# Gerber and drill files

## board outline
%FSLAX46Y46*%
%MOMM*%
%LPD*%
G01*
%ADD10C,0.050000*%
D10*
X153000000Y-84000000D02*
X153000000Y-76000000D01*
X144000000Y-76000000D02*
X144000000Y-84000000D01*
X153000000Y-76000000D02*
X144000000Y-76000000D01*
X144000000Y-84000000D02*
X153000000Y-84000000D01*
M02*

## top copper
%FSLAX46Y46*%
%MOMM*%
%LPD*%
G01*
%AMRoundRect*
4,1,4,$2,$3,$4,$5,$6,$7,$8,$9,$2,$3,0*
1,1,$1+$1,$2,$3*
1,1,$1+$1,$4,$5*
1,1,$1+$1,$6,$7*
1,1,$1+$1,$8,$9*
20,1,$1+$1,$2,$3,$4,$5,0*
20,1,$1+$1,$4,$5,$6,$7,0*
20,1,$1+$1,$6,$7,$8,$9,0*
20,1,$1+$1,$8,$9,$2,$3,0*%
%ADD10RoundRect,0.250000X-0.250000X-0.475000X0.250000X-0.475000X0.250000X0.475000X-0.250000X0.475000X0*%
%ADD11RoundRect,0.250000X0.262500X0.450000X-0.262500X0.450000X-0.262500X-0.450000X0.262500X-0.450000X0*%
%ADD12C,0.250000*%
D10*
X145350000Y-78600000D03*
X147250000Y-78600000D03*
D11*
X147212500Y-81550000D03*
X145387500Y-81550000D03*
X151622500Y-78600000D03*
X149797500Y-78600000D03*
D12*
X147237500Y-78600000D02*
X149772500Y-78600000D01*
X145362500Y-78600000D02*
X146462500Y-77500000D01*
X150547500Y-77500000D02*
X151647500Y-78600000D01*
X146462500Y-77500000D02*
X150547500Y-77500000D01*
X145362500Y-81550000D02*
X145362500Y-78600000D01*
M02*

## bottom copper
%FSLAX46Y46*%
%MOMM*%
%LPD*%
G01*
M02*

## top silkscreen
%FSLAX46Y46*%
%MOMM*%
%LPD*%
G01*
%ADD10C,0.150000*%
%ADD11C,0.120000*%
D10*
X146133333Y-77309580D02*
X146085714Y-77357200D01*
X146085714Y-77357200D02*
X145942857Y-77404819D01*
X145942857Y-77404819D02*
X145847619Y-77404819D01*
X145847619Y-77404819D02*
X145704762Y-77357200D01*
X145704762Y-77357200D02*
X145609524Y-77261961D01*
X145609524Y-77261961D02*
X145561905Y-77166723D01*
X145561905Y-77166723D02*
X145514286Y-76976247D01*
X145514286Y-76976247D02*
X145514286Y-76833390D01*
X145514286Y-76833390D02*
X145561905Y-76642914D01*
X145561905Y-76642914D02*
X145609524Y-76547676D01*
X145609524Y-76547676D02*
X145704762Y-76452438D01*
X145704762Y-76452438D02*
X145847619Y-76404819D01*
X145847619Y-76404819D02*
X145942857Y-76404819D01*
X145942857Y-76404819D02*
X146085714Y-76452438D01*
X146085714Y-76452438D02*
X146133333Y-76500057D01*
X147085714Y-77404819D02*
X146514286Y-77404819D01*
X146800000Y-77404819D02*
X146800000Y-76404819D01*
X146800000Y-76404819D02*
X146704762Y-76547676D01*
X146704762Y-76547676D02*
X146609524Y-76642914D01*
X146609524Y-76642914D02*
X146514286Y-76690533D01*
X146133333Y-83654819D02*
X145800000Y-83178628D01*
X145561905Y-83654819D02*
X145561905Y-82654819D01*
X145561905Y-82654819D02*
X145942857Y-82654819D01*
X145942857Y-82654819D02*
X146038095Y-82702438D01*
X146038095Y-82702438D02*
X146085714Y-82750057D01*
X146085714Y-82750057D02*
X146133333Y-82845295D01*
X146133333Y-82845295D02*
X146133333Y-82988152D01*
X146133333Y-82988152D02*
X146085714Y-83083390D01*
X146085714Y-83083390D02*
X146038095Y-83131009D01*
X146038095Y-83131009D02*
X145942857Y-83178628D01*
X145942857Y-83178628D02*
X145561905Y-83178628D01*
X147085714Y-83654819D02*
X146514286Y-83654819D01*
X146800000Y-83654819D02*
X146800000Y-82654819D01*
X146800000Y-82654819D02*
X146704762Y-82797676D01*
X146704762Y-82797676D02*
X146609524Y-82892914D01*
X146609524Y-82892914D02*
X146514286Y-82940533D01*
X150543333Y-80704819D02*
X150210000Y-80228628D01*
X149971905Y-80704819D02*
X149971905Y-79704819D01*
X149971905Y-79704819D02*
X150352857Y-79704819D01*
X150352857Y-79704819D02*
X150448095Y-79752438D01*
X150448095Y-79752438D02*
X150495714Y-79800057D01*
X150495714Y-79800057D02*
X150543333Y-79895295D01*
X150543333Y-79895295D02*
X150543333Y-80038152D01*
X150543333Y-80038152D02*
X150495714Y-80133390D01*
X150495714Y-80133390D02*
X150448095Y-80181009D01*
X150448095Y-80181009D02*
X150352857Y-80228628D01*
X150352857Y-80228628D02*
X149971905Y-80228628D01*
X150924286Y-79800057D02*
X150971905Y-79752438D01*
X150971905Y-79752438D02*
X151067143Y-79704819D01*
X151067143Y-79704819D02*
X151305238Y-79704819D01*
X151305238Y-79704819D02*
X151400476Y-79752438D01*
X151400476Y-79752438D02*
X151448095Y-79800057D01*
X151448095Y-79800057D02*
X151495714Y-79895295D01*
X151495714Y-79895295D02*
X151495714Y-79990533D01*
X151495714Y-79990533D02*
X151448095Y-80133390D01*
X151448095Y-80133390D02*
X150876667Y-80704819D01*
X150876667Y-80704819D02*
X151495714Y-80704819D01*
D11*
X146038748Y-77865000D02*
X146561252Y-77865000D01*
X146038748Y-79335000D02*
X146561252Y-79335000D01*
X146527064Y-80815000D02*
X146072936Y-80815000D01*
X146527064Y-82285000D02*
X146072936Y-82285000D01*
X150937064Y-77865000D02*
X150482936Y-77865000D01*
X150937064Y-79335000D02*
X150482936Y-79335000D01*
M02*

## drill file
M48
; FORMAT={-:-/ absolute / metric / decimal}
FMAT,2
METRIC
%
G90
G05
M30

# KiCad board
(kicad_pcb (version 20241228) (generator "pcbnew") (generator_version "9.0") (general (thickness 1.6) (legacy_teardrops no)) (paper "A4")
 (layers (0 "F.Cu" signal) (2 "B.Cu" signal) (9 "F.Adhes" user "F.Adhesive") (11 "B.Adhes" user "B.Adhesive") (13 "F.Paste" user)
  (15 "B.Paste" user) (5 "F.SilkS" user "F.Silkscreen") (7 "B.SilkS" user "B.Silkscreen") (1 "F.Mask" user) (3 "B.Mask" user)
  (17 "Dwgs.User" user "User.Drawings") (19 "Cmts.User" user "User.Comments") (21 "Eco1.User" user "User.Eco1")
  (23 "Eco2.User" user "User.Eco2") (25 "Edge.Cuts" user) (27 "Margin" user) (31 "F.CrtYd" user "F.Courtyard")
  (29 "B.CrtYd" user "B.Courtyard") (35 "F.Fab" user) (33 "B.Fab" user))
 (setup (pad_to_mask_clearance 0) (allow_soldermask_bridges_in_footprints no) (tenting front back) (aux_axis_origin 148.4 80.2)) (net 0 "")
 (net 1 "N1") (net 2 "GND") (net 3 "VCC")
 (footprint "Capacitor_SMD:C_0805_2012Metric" (layer "F.Cu") (at 146.3 78.6)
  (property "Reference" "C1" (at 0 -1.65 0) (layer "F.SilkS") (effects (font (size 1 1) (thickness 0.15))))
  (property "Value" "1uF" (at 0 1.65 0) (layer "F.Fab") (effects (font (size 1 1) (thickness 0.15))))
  (fp_line (start -0.261252 -0.735) (end 0.261252 -0.735) (stroke (width 0.12) (type solid)) (layer "F.SilkS"))
  (fp_line (start -0.261252 0.735) (end 0.261252 0.735) (stroke (width 0.12) (type solid)) (layer "F.SilkS"))
  (pad "1" smd roundrect (at -0.95 0) (size 1 1.45) (layers "F.Cu" "F.Mask" "F.Paste") (roundrect_rratio 0.25) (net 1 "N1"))
  (pad "2" smd roundrect (at 0.95 0) (size 1 1.45) (layers "F.Cu" "F.Mask" "F.Paste") (roundrect_rratio 0.25) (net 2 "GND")))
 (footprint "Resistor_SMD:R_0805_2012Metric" (layer "F.Cu") (at 146.3 81.55 180)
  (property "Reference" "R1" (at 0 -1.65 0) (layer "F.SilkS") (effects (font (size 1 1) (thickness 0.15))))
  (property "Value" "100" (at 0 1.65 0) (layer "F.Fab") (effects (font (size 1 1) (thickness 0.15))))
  (fp_line (start -0.227064 0.735) (end 0.227064 0.735) (stroke (width 0.12) (type solid)) (layer "F.SilkS"))
  (fp_line (start -0.227064 -0.735) (end 0.227064 -0.735) (stroke (width 0.12) (type solid)) (layer "F.SilkS"))
  (pad "1" smd roundrect (at -0.9125 0 180) (size 1.025 1.4) (layers "F.Cu" "F.Mask" "F.Paste") (roundrect_rratio 0.243902) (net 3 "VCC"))
  (pad "2" smd roundrect (at 0.9125 0 180) (size 1.025 1.4) (layers "F.Cu" "F.Mask" "F.Paste") (roundrect_rratio 0.243902) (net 1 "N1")))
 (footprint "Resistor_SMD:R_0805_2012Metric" (layer "F.Cu") (at 150.71 78.6 180)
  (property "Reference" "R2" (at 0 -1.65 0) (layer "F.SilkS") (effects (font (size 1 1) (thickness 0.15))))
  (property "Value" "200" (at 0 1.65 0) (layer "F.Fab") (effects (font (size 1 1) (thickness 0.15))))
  (fp_line (start -0.227064 0.735) (end 0.227064 0.735) (stroke (width 0.12) (type solid)) (layer "F.SilkS"))
  (fp_line (start -0.227064 -0.735) (end 0.227064 -0.735) (stroke (width 0.12) (type solid)) (layer "F.SilkS"))
  (pad "1" smd roundrect (at -0.9125 0 180) (size 1.025 1.4) (layers "F.Cu" "F.Mask" "F.Paste") (roundrect_rratio 0.243902) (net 1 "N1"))
  (pad "2" smd roundrect (at 0.9125 0 180) (size 1.025 1.4) (layers "F.Cu" "F.Mask" "F.Paste") (roundrect_rratio 0.243902) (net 2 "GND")))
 (gr_line (start 153 84) (end 153 76) (stroke (width 0.05) (type solid)) (layer "Edge.Cuts"))
 (gr_line (start 144 76) (end 144 84) (stroke (width 0.05) (type solid)) (layer "Edge.Cuts"))
 (gr_line (start 153 76) (end 144 76) (stroke (width 0.05) (type solid)) (layer "Edge.Cuts"))
 (gr_line (start 144 84) (end 153 84) (stroke (width 0.05) (type solid)) (layer "Edge.Cuts"))
 (segment (start 147.2375 78.6) (end 149.7725 78.6) (width 0.25) (layer "F.Cu") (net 2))
 (segment (start 145.3625 78.6) (end 146.4625 77.5) (width 0.25) (layer "F.Cu") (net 1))
 (segment (start 150.5475 77.5) (end 151.6475 78.6) (width 0.25) (layer "F.Cu") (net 1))
 (segment (start 146.4625 77.5) (end 150.5475 77.5) (width 0.25) (layer "F.Cu") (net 1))
 (segment (start 145.3625 81.55) (end 145.3625 78.6) (width 0.25) (layer "F.Cu") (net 1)))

